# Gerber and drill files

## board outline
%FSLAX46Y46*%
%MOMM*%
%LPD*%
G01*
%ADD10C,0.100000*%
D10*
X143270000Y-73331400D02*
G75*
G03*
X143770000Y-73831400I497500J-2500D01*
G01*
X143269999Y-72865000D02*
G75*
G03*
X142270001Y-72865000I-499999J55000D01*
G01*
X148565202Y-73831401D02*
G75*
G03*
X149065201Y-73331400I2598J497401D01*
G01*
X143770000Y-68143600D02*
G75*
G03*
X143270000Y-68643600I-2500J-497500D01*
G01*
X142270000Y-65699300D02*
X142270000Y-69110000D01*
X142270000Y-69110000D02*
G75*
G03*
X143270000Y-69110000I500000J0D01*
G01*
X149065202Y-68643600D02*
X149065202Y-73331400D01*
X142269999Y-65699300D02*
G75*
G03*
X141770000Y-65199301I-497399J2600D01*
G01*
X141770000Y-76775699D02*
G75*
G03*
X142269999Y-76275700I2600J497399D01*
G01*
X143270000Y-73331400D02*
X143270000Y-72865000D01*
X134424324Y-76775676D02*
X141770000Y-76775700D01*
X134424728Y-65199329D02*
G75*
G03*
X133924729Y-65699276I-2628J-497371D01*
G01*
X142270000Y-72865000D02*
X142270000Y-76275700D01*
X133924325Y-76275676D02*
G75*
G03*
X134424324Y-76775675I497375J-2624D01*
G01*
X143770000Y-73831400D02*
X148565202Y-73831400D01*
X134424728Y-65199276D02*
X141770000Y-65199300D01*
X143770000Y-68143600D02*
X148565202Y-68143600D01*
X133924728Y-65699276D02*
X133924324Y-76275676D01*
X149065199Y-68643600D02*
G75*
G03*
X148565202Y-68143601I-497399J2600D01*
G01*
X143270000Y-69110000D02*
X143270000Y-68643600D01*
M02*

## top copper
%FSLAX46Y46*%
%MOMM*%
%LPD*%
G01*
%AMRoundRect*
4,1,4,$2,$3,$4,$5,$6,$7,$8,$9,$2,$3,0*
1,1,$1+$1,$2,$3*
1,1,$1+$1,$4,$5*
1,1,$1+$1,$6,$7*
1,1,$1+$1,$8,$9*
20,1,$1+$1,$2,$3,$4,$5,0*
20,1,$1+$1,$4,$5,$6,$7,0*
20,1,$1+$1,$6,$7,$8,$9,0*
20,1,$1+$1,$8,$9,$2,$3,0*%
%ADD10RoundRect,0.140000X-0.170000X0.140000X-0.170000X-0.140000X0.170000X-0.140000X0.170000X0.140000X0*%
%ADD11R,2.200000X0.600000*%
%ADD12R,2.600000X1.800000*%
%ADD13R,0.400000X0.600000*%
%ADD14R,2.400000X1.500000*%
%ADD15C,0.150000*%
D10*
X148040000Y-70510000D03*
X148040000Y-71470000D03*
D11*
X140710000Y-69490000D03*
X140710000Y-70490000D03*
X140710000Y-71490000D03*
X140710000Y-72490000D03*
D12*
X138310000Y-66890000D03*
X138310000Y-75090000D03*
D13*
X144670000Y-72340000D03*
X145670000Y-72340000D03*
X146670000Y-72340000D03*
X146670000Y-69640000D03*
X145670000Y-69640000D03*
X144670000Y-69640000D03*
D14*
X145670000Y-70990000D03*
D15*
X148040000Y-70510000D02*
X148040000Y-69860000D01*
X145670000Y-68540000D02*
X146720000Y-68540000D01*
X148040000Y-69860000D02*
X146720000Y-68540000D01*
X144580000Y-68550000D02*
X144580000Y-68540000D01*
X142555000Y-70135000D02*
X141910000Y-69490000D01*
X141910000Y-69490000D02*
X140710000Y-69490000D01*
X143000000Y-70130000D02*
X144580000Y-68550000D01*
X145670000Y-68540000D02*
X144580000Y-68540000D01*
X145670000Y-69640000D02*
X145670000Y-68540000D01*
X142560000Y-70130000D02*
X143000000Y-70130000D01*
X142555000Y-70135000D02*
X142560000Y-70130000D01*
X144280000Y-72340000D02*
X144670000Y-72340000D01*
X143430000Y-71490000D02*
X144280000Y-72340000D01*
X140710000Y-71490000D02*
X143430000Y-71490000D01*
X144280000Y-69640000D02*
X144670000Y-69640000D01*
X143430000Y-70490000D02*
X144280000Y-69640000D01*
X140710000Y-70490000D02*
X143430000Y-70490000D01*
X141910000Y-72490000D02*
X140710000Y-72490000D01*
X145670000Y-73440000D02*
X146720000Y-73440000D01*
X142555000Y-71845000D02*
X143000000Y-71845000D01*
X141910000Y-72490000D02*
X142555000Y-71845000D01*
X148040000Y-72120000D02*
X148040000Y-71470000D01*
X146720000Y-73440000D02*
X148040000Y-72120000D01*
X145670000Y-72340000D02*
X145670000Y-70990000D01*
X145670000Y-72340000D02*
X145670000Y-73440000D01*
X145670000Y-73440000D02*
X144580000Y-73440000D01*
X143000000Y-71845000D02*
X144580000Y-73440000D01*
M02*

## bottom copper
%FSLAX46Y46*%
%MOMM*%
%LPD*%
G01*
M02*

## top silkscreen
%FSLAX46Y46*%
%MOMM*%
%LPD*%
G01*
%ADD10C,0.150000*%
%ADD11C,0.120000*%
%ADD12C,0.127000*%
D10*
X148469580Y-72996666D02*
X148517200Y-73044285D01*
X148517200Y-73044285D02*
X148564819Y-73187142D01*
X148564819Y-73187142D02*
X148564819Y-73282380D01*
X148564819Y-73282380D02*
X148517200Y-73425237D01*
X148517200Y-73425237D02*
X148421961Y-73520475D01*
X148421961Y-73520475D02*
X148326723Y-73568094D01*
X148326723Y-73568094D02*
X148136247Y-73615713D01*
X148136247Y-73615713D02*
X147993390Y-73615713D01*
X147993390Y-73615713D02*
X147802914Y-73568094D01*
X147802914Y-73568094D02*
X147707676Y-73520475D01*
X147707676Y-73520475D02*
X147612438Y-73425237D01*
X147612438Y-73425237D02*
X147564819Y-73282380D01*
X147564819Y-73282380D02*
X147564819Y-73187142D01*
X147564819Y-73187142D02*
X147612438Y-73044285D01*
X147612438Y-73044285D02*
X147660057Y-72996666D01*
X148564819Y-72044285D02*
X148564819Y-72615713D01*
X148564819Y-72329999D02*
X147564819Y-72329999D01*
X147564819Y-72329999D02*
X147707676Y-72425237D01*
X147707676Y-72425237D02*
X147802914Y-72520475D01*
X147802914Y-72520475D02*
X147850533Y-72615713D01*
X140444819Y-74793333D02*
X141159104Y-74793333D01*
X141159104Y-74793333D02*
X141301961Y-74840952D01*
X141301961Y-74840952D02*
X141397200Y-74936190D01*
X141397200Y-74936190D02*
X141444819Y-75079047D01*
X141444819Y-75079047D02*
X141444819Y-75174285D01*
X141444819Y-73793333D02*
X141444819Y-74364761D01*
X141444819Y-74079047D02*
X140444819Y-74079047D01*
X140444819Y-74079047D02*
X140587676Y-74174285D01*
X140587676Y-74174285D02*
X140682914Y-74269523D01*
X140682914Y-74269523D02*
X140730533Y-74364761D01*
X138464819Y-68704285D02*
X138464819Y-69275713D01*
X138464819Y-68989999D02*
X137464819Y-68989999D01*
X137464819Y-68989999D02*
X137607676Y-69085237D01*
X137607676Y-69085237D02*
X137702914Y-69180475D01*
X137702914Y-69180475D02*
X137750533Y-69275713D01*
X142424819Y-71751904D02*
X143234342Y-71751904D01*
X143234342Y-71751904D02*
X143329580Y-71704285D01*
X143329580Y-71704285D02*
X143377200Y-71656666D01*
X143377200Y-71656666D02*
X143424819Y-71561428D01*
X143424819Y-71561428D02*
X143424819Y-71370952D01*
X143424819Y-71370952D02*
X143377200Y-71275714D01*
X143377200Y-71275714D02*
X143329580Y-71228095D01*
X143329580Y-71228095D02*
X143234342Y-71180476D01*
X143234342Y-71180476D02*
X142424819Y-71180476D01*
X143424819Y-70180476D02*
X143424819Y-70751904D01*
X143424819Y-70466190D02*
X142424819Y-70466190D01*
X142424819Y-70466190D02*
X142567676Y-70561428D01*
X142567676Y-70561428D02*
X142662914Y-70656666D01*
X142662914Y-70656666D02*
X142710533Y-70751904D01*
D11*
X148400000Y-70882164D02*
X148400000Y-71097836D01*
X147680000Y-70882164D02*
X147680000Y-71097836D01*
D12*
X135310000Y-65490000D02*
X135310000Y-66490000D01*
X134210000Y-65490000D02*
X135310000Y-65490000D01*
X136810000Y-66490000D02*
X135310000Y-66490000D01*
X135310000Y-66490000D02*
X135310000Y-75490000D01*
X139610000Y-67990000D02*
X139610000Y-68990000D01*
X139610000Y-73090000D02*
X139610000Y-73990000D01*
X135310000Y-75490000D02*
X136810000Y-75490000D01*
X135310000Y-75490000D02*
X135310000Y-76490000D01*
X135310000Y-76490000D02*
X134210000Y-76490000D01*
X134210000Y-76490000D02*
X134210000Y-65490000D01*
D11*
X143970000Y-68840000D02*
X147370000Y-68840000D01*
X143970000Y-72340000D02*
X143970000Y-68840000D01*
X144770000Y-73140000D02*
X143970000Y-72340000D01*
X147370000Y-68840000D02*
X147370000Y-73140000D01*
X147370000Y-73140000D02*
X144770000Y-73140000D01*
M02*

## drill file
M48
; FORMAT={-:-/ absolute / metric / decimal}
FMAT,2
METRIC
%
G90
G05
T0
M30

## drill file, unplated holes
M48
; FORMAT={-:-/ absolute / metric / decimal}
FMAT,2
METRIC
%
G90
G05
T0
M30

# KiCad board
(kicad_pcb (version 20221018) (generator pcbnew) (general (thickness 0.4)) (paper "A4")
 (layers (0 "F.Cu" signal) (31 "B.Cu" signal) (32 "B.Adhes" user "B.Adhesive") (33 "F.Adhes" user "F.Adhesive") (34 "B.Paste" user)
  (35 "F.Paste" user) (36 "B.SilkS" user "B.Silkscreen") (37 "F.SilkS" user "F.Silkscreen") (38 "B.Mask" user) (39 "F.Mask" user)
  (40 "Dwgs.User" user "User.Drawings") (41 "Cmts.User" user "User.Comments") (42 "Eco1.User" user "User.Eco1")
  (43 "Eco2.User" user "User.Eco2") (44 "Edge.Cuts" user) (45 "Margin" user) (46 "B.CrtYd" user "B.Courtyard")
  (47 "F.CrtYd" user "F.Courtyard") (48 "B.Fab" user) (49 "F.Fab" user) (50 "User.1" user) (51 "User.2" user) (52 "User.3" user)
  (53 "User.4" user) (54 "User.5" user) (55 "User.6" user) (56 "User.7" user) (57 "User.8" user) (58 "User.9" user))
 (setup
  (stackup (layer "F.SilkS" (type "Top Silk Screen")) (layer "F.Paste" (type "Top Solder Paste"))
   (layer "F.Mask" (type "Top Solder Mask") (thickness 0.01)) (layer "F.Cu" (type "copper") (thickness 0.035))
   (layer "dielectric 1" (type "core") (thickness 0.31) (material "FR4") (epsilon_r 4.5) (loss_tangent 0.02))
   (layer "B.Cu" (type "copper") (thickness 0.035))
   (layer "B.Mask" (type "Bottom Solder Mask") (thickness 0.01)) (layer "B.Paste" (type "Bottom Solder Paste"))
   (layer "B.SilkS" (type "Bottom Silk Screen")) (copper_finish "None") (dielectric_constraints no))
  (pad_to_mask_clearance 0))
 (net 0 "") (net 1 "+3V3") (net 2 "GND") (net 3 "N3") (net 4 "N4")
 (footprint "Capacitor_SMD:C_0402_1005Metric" (layer "F.Cu") (at 148.04 70.99 -90)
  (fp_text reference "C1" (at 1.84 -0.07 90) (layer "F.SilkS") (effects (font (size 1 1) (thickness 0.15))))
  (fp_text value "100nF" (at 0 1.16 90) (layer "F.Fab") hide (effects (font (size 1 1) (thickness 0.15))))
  (fp_line (start -0.107836 -0.36) (end 0.107836 -0.36) (stroke (width 0.12) (type solid)) (layer "F.SilkS"))
  (fp_line (start -0.107836 0.36) (end 0.107836 0.36) (stroke (width 0.12) (type solid)) (layer "F.SilkS"))
  (pad "1" smd roundrect (at -0.48 0 270) (size 0.56 0.62) (layers "F.Cu" "F.Paste" "F.Mask") (roundrect_rratio 0.25) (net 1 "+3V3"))
  (pad "2" smd roundrect (at 0.48 0 270) (size 0.56 0.62) (layers "F.Cu" "F.Paste" "F.Mask") (roundrect_rratio 0.25) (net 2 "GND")))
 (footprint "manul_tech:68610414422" (layer "F.Cu") (at 138.31 70.99 -90)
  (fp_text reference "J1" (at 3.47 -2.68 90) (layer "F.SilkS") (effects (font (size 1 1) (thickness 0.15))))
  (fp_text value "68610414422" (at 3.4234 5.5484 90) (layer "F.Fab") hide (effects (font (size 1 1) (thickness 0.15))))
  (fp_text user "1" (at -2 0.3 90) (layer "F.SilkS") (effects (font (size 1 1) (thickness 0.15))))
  (fp_line (start -5.5 3) (end -4.5 3) (stroke (width 0.127) (type solid)) (layer "F.SilkS"))
  (fp_line (start -5.5 4.1) (end -5.5 3) (stroke (width 0.127) (type solid)) (layer "F.SilkS"))
  (fp_line (start -4.5 1.5) (end -4.5 3) (stroke (width 0.127) (type solid)) (layer "F.SilkS"))
  (fp_line (start -4.5 3) (end 4.5 3) (stroke (width 0.127) (type solid)) (layer "F.SilkS"))
  (fp_line (start -3 -1.3) (end -2 -1.3) (stroke (width 0.127) (type solid)) (layer "F.SilkS"))
  (fp_line (start 2.1 -1.3) (end 3 -1.3) (stroke (width 0.127) (type solid)) (layer "F.SilkS"))
  (fp_line (start 4.5 3) (end 4.5 1.5) (stroke (width 0.127) (type solid)) (layer "F.SilkS"))
  (fp_line (start 4.5 3) (end 5.5 3) (stroke (width 0.127) (type solid)) (layer "F.SilkS"))
  (fp_line (start 5.5 3) (end 5.5 4.1) (stroke (width 0.127) (type solid)) (layer "F.SilkS"))
  (fp_line (start 5.5 4.1) (end -5.5 4.1) (stroke (width 0.127) (type solid)) (layer "F.SilkS"))
  (pad "1" smd rect (at -1.5 -2.4 270) (size 0.6 2.2) (layers "F.Cu" "F.Paste" "F.Mask") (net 1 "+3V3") (solder_mask_margin 0.102))
  (pad "2" smd rect (at -0.5 -2.4 270) (size 0.6 2.2) (layers "F.Cu" "F.Paste" "F.Mask") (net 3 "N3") (solder_mask_margin 0.102))
  (pad "3" smd rect (at 0.5 -2.4 270) (size 0.6 2.2) (layers "F.Cu" "F.Paste" "F.Mask") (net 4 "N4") (solder_mask_margin 0.102))
  (pad "4" smd rect (at 1.5 -2.4 270) (size 0.6 2.2) (layers "F.Cu" "F.Paste" "F.Mask") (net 2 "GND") (solder_mask_margin 0.102))
  (pad "Z1" smd rect (at -4.1 0 270) (size 1.8 2.6) (layers "F.Cu" "F.Paste" "F.Mask") (solder_mask_margin 0.102))
  (pad "Z2" smd rect (at 4.1 0 270) (size 1.8 2.6) (layers "F.Cu" "F.Paste" "F.Mask") (solder_mask_margin 0.102)))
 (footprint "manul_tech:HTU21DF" (layer "F.Cu") (at 145.67 70.99)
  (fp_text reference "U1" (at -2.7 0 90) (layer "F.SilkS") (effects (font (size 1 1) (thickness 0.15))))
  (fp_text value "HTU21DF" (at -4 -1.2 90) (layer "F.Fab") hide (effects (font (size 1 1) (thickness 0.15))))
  (fp_line (start -1.7 -2.15) (end 1.7 -2.15) (stroke (width 0.12) (type solid)) (layer "F.SilkS"))
  (fp_line (start -1.7 1.35) (end -1.7 -2.15) (stroke (width 0.12) (type solid)) (layer "F.SilkS"))
  (fp_line (start -0.9 2.15) (end -1.7 1.35) (stroke (width 0.12) (type solid)) (layer "F.SilkS"))
  (fp_line (start 1.7 -2.15) (end 1.7 2.15) (stroke (width 0.12) (type solid)) (layer "F.SilkS"))
  (fp_line (start 1.7 2.15) (end -0.9 2.15) (stroke (width 0.12) (type solid)) (layer "F.SilkS"))
  (pad "1" smd rect (at -1 1.35) (size 0.4 0.6) (layers "F.Cu" "F.Paste" "F.Mask") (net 4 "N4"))
  (pad "2" smd rect (at 0 1.35) (size 0.4 0.6) (layers "F.Cu" "F.Paste" "F.Mask") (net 2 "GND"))
  (pad "3" smd rect (at 1 1.35) (size 0.4 0.6) (layers "F.Cu" "F.Paste" "F.Mask"))
  (pad "4" smd rect (at 1 -1.35) (size 0.4 0.6) (layers "F.Cu" "F.Paste" "F.Mask"))
  (pad "5" smd rect (at 0 -1.35) (size 0.4 0.6) (layers "F.Cu" "F.Paste" "F.Mask") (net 1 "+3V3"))
  (pad "6" smd rect (at -1 -1.35) (size 0.4 0.6) (layers "F.Cu" "F.Paste" "F.Mask") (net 3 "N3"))
  (pad "7" smd rect (at 0 0 90) (size 1.5 2.4) (layers "F.Cu" "F.Paste" "F.Mask") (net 2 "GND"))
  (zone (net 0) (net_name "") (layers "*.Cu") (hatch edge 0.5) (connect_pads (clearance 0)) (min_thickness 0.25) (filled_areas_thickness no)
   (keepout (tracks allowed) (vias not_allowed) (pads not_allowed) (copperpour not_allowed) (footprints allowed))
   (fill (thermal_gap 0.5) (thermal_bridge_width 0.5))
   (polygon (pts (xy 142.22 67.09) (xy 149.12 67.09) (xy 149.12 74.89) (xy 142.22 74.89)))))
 (gr_arc (start 143.77 73.8314) (mid 143.415713 73.685687) (end 143.27 73.3314) (stroke (width 0.1) (type default)) (layer "Edge.Cuts"))
 (gr_arc (start 142.27 72.865) (mid 142.77 72.306984) (end 143.27 72.865) (stroke (width 0.1) (type default)) (layer "Edge.Cuts"))
 (gr_arc (start 149.065202 73.3314) (mid 148.919526 73.685724) (end 148.565202 73.8314) (stroke (width 0.1) (type default))
  (layer "Edge.Cuts"))
 (gr_arc (start 143.27 68.6436) (mid 143.415713 68.289313) (end 143.77 68.1436) (stroke (width 0.1) (type default)) (layer "Edge.Cuts"))
 (gr_line (start 142.27 65.6993) (end 142.27 69.11) (stroke (width 0.1) (type default)) (layer "Edge.Cuts"))
 (gr_arc (start 143.27 69.11) (mid 142.77 69.61) (end 142.27 69.11) (stroke (width 0.1) (type default)) (layer "Edge.Cuts"))
 (gr_line (start 149.065202 68.6436) (end 149.065202 73.3314) (stroke (width 0.1) (type default)) (layer "Edge.Cuts"))
 (gr_arc (start 141.77 65.1993) (mid 142.124324 65.344976) (end 142.27 65.6993) (stroke (width 0.1) (type default)) (layer "Edge.Cuts"))
 (gr_arc (start 142.27 76.2757) (mid 142.124324 76.630024) (end 141.77 76.7757) (stroke (width 0.1) (type default)) (layer "Edge.Cuts"))
 (gr_line (start 143.27 73.3314) (end 143.27 72.865) (stroke (width 0.1) (type default)) (layer "Edge.Cuts"))
 (gr_line (start 134.424324 76.775676) (end 141.77 76.7757) (stroke (width 0.1) (type default)) (layer "Edge.Cuts"))
 (gr_arc (start 133.924728 65.699276) (mid 134.070404 65.344952) (end 134.424728 65.199276) (stroke (width 0.1) (type default))
  (layer "Edge.Cuts"))
 (gr_line (start 142.27 72.865) (end 142.27 76.2757) (stroke (width 0.1) (type default)) (layer "Edge.Cuts"))
 (gr_arc (start 134.424324 76.775676) (mid 134.07 76.63) (end 133.924324 76.275676) (stroke (width 0.1) (type default)) (layer "Edge.Cuts"))
 (gr_line (start 143.77 73.8314) (end 148.565202 73.8314) (stroke (width 0.1) (type default)) (layer "Edge.Cuts"))
 (gr_line (start 134.424728 65.199276) (end 141.77 65.1993) (stroke (width 0.1) (type default)) (layer "Edge.Cuts"))
 (gr_line (start 143.77 68.1436) (end 148.565202 68.1436) (stroke (width 0.1) (type default)) (layer "Edge.Cuts"))
 (gr_line (start 133.924728 65.699276) (end 133.924324 76.275676) (stroke (width 0.1) (type default)) (layer "Edge.Cuts"))
 (gr_arc (start 148.565202 68.1436) (mid 148.919526 68.289276) (end 149.065202 68.6436) (stroke (width 0.1) (type default))
  (layer "Edge.Cuts"))
 (gr_line (start 143.27 69.11) (end 143.27 68.6436) (stroke (width 0.1) (type default)) (layer "Edge.Cuts"))
 (segment (start 148.04 70.51) (end 148.04 69.86) (width 0.15) (layer "F.Cu") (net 1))
 (segment (start 145.67 68.54) (end 146.72 68.54) (width 0.15) (layer "F.Cu") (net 1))
 (segment (start 148.04 69.86) (end 146.72 68.54) (width 0.15) (layer "F.Cu") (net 1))
 (segment (start 144.58 68.55) (end 144.58 68.54) (width 0.15) (layer "F.Cu") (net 1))
 (segment (start 142.555 70.135) (end 141.91 69.49) (width 0.15) (layer "F.Cu") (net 1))
 (segment (start 141.91 69.49) (end 140.71 69.49) (width 0.15) (layer "F.Cu") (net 1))
 (segment (start 143 70.13) (end 144.58 68.55) (width 0.15) (layer "F.Cu") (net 1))
 (segment (start 145.67 68.54) (end 144.58 68.54) (width 0.15) (layer "F.Cu") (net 1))
 (segment (start 145.67 69.64) (end 145.67 68.54) (width 0.15) (layer "F.Cu") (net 1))
 (segment (start 142.56 70.13) (end 143 70.13) (width 0.15) (layer "F.Cu") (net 1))
 (segment (start 142.555 70.135) (end 142.56 70.13) (width 0.15) (layer "F.Cu") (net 1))
 (segment (start 144.28 72.34) (end 144.67 72.34) (width 0.15) (layer "F.Cu") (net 4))
 (segment (start 143.43 71.49) (end 144.28 72.34) (width 0.15) (layer "F.Cu") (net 4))
 (segment (start 140.71 71.49) (end 143.43 71.49) (width 0.15) (layer "F.Cu") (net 4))
 (segment (start 144.28 69.64) (end 144.67 69.64) (width 0.15) (layer "F.Cu") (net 3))
 (segment (start 143.43 70.49) (end 144.28 69.64) (width 0.15) (layer "F.Cu") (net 3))
 (segment (start 140.71 70.49) (end 143.43 70.49) (width 0.15) (layer "F.Cu") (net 3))
 (segment (start 141.91 72.49) (end 140.71 72.49) (width 0.15) (layer "F.Cu") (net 2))
 (segment (start 145.67 73.44) (end 146.72 73.44) (width 0.15) (layer "F.Cu") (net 2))
 (segment (start 142.555 71.845) (end 143 71.845) (width 0.15) (layer "F.Cu") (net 2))
 (segment (start 141.91 72.49) (end 142.555 71.845) (width 0.15) (layer "F.Cu") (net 2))
 (segment (start 148.04 72.12) (end 148.04 71.47) (width 0.15) (layer "F.Cu") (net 2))
 (segment (start 146.72 73.44) (end 148.04 72.12) (width 0.15) (layer "F.Cu") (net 2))
 (segment (start 145.67 72.34) (end 145.67 70.99) (width 0.15) (layer "F.Cu") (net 2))
 (segment (start 145.67 72.34) (end 145.67 73.44) (width 0.15) (layer "F.Cu") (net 2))
 (segment (start 145.67 73.44) (end 144.58 73.44) (width 0.15) (layer "F.Cu") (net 2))
 (segment (start 143 71.845) (end 144.58 73.44) (width 0.15) (layer "F.Cu") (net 2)))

